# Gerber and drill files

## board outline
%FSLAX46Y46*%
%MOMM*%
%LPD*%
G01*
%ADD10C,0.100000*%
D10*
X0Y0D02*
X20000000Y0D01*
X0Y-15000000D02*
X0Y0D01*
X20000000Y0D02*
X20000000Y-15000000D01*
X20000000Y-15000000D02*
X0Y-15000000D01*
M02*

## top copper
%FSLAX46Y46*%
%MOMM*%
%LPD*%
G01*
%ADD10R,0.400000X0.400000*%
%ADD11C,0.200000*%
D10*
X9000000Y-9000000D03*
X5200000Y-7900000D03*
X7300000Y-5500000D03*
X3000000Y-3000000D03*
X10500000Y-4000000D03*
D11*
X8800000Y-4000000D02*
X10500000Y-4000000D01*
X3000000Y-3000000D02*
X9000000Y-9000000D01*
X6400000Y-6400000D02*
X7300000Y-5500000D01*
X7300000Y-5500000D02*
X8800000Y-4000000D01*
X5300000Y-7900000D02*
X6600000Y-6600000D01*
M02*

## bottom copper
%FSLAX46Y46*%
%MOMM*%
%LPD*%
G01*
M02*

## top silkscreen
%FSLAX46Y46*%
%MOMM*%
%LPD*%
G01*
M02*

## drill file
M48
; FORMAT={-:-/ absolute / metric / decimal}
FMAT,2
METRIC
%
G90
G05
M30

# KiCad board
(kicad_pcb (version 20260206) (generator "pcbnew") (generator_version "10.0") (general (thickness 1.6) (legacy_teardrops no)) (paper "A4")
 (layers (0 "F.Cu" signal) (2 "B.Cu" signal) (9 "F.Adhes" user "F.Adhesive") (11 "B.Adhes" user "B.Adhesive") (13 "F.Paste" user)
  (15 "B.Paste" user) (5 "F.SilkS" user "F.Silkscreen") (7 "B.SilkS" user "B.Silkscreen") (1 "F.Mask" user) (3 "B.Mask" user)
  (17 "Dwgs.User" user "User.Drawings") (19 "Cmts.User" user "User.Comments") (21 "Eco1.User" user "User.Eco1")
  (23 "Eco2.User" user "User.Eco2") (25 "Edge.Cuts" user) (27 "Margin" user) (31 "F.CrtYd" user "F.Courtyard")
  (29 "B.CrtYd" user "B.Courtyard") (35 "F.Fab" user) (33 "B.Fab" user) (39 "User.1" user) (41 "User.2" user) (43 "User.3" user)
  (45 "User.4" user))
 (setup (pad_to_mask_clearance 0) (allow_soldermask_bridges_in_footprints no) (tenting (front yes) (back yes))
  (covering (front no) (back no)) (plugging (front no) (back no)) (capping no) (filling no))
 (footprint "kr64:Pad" (layer "F.Cu") (at 9 9)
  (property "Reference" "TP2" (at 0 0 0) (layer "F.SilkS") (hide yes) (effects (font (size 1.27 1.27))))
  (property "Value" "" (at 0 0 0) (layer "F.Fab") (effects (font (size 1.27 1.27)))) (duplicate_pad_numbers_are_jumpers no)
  (pad "1" smd rect (at 0 0) (size 0.4 0.4) (layers "F.Cu" "F.Mask" "F.Paste") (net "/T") (thermal_bridge_angle 45)))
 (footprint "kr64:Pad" (layer "F.Cu") (at 5.2 7.9)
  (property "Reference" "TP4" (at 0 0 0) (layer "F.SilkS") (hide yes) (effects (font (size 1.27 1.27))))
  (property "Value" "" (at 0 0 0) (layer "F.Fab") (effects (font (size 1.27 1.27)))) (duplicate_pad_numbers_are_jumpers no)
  (pad "1" smd rect (at 0 0) (size 0.4 0.4) (layers "F.Cu" "F.Mask" "F.Paste") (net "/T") (thermal_bridge_angle 45)))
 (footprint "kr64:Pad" (layer "F.Cu") (at 7.3 5.5)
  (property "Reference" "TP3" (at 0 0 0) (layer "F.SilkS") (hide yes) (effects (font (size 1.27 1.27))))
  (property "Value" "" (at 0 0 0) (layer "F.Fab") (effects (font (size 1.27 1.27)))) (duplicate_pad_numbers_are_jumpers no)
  (pad "1" smd rect (at 0 0) (size 0.4 0.4) (layers "F.Cu" "F.Mask" "F.Paste") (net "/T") (thermal_bridge_angle 45)))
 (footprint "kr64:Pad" (layer "F.Cu") (at 3 3)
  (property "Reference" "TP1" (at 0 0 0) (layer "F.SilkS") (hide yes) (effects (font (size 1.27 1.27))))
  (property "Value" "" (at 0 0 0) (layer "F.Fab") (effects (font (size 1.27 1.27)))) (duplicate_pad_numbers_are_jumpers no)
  (pad "1" smd rect (at 0 0) (size 0.4 0.4) (layers "F.Cu" "F.Mask" "F.Paste") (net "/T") (thermal_bridge_angle 45)))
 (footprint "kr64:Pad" (layer "F.Cu") (at 10.5 4)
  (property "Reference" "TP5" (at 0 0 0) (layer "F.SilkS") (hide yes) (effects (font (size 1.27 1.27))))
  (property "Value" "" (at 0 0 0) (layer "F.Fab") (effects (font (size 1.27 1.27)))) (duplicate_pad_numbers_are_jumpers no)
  (pad "1" smd rect (at 0 0) (size 0.4 0.4) (layers "F.Cu" "F.Mask" "F.Paste") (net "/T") (thermal_bridge_angle 45)))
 (gr_line (start 0 0) (end 20 0) (stroke (width 0.1) (type default)) (layer "Edge.Cuts"))
 (gr_line (start 0 15) (end 0 0) (stroke (width 0.1) (type default)) (layer "Edge.Cuts"))
 (gr_line (start 20 0) (end 20 15) (stroke (width 0.1) (type default)) (layer "Edge.Cuts"))
 (gr_line (start 20 15) (end 0 15) (stroke (width 0.1) (type default)) (layer "Edge.Cuts"))
 (segment (start 8.8 4) (end 10.5 4) (width 0.2) (layer "F.Cu") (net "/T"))
 (segment (start 3 3) (end 9 9) (width 0.2) (layer "F.Cu") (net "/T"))
 (segment (start 6.4 6.4) (end 7.3 5.5) (width 0.2) (layer "F.Cu") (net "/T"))
 (segment (start 7.3 5.5) (end 8.8 4) (width 0.2) (layer "F.Cu") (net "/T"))
 (segment (start 5.3 7.9) (end 6.6 6.6) (width 0.2) (layer "F.Cu") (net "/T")))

